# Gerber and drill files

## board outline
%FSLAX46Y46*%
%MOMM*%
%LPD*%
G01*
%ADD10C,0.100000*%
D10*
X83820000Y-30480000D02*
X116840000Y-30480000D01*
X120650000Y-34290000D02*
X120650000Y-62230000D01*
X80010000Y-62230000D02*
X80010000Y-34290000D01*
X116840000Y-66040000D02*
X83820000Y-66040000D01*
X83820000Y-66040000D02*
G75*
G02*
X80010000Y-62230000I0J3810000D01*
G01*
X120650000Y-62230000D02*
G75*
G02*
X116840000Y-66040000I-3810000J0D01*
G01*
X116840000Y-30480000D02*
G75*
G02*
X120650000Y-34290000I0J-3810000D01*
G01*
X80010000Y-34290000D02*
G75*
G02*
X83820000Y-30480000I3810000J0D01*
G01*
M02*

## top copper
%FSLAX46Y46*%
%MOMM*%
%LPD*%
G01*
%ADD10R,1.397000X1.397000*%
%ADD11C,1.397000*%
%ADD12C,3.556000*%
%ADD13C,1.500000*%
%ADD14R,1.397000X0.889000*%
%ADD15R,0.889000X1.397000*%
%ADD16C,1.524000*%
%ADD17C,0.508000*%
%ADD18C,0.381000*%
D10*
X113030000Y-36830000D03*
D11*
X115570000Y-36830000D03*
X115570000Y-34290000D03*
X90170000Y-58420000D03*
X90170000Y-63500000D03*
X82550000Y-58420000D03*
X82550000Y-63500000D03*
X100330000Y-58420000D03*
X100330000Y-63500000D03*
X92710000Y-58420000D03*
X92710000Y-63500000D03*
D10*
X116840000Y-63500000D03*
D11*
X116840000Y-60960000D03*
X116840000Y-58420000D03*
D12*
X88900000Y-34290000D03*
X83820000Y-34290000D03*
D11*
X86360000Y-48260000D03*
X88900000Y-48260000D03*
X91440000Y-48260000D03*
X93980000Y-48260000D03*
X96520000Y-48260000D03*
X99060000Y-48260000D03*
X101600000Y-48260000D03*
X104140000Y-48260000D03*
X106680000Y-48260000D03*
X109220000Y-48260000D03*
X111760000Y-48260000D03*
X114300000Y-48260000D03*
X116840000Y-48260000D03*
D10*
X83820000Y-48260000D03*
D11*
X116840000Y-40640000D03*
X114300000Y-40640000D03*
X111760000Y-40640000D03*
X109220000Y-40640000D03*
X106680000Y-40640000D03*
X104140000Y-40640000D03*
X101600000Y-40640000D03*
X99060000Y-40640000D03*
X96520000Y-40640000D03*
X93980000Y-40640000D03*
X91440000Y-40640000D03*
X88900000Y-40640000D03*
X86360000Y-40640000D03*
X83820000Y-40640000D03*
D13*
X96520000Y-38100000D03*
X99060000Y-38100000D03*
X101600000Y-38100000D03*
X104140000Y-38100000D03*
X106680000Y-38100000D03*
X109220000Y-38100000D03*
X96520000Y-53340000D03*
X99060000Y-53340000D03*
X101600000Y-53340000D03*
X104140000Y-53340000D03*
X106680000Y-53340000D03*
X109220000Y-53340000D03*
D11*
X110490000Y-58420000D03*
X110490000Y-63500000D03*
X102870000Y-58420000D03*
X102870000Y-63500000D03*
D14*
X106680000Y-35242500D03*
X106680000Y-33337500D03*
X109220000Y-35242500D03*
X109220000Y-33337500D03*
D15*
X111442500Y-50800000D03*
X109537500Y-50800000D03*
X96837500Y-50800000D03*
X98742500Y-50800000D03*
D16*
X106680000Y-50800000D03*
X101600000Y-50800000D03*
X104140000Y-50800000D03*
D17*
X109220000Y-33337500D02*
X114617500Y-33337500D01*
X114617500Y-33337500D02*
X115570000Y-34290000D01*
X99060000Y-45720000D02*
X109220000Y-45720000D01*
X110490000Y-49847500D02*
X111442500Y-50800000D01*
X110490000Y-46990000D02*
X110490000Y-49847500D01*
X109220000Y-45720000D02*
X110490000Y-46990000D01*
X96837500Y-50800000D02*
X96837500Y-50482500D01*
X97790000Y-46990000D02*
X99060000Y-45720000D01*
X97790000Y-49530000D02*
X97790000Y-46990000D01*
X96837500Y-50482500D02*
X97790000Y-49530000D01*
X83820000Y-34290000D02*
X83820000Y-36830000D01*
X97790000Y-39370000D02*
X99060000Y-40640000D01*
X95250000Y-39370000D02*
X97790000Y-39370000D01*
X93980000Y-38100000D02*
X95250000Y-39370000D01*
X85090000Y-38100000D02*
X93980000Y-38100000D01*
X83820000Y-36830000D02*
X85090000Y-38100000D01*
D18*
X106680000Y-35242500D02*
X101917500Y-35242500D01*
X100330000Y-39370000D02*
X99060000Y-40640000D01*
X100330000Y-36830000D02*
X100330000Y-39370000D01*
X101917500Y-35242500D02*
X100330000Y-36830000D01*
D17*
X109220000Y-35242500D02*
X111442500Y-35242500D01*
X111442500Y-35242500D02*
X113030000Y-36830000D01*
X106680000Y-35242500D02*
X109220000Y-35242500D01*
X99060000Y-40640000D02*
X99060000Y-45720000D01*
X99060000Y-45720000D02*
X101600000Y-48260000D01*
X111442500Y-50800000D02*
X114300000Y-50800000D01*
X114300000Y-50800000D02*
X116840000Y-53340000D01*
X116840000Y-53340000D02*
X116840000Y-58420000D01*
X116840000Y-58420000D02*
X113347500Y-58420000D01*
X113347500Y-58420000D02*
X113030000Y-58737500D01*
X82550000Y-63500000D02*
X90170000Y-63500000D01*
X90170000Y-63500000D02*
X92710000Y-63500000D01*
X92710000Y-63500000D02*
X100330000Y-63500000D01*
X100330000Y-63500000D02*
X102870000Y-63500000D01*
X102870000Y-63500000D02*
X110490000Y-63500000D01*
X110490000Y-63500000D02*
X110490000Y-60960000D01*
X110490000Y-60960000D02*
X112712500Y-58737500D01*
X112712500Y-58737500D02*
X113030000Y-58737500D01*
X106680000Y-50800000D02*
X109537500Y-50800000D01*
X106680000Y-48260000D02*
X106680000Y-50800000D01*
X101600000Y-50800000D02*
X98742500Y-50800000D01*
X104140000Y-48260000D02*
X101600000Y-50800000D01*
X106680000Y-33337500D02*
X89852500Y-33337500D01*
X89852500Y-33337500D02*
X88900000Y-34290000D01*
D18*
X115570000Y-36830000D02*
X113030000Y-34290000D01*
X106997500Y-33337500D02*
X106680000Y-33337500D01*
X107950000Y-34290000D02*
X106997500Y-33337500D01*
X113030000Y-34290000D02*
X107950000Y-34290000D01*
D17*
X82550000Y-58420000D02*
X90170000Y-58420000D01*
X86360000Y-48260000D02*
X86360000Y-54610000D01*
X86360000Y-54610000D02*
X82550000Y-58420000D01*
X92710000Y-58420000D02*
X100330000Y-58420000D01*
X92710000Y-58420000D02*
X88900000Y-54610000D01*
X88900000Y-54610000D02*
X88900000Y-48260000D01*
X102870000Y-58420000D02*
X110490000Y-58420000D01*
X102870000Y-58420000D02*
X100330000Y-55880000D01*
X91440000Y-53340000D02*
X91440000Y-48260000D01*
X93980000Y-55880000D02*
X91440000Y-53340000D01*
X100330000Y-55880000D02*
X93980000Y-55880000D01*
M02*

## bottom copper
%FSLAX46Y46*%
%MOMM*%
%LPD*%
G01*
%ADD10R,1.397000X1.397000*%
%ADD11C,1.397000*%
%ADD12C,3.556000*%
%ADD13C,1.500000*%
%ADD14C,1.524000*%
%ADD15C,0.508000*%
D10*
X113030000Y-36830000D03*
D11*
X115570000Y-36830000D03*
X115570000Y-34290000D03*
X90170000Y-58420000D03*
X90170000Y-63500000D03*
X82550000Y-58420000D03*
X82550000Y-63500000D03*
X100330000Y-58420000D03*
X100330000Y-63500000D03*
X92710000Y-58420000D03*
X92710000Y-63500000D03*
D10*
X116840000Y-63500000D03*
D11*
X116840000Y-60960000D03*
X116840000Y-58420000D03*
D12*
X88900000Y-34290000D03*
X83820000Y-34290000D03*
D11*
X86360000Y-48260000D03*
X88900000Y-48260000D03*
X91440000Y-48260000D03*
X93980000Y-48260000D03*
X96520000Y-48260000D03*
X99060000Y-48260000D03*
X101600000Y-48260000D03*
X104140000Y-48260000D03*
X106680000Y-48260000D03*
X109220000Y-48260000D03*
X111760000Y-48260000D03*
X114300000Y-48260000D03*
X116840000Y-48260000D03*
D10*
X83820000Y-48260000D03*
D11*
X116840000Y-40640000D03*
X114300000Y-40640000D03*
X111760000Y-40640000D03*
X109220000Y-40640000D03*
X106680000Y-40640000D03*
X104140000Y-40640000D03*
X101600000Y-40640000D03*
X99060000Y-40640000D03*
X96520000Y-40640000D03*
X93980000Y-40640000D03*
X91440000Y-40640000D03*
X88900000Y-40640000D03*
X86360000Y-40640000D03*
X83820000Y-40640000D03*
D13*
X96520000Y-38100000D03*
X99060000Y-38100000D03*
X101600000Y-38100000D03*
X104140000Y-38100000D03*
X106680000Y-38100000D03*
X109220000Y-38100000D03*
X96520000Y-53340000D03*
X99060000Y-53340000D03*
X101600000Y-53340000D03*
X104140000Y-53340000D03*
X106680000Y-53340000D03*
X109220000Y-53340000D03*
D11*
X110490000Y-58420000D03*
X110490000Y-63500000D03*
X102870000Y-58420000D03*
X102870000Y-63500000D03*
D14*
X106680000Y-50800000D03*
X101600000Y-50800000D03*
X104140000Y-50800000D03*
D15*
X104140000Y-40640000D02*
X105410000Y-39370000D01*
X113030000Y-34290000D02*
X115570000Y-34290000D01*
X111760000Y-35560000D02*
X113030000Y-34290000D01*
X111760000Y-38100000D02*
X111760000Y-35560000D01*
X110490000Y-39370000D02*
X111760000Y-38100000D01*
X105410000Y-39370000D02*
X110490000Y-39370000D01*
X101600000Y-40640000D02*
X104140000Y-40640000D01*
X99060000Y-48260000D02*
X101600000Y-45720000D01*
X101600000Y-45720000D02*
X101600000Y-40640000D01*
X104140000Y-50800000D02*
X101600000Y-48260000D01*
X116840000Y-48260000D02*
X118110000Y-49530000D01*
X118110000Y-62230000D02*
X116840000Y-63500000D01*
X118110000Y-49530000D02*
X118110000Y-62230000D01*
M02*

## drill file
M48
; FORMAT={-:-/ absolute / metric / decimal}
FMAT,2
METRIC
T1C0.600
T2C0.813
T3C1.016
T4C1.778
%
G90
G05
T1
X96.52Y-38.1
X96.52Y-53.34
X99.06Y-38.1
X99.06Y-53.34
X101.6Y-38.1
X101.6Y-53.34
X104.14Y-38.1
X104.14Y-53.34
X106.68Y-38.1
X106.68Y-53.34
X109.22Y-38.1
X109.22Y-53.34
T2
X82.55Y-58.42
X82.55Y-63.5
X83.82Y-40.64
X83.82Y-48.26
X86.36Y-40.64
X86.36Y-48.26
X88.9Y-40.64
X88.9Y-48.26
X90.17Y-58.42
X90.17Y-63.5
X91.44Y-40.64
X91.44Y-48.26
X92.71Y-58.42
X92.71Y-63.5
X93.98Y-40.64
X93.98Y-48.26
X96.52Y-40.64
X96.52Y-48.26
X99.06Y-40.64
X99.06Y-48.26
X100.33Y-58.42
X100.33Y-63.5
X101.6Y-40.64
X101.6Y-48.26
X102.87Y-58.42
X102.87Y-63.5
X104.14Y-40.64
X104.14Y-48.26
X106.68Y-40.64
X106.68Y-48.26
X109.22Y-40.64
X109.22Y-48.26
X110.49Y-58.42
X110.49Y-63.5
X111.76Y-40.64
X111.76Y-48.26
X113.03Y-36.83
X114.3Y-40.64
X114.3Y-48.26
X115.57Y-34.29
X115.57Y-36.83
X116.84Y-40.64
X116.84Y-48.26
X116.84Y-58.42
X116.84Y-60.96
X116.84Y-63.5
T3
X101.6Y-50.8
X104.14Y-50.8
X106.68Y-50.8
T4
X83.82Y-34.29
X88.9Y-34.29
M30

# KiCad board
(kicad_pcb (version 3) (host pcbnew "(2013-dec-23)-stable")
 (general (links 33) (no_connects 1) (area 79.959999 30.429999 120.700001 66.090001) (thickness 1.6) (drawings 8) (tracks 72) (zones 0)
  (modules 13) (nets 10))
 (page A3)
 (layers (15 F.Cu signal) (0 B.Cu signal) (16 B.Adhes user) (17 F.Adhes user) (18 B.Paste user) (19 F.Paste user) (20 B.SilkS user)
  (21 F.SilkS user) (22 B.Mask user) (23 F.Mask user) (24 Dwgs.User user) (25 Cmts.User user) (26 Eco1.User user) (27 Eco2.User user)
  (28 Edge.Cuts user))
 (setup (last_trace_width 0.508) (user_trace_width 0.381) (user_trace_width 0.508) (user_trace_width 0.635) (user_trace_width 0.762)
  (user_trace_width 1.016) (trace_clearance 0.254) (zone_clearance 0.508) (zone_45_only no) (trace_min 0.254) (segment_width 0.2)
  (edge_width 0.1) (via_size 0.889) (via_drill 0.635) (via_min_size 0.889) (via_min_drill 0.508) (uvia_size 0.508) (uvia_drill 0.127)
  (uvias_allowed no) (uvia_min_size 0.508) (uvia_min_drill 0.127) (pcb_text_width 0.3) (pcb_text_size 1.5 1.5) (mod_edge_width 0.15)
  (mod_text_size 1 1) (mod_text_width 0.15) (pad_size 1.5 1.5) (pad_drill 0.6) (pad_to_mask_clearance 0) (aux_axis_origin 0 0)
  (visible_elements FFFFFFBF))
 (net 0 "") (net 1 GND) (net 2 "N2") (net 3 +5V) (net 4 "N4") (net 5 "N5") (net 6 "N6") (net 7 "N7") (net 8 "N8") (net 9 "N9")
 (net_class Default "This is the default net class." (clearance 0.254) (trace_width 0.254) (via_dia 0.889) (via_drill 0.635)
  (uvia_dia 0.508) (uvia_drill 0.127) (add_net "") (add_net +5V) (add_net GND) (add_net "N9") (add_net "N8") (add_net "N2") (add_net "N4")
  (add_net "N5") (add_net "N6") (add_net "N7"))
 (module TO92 (layer F.Cu) (at 114.3 35.56 180)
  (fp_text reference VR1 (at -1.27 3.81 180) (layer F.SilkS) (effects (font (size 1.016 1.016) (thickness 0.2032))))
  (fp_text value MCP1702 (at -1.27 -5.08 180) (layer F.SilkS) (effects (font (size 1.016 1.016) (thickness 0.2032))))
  (pad 1 thru_hole rect (at 1.27 -1.27 180) (size 1.397 1.397) (drill 0.8128) (layers *.Cu *.Mask F.SilkS) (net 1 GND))
  (pad 2 thru_hole circle (at -1.27 -1.27 180) (size 1.397 1.397) (drill 0.8128) (layers *.Cu *.Mask F.SilkS) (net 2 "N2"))
  (pad 3 thru_hole circle (at -1.27 1.27 180) (size 1.397 1.397) (drill 0.8128) (layers *.Cu *.Mask F.SilkS) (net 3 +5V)))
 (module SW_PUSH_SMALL (layer F.Cu) (at 86.36 60.96)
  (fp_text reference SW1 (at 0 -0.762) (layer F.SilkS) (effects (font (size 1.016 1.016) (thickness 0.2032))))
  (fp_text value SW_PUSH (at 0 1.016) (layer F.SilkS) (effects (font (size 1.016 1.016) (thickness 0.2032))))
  (pad 1 thru_hole circle (at 3.81 -2.54) (size 1.397 1.397) (drill 0.8128) (layers *.Cu *.Mask F.SilkS) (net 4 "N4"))
  (pad 2 thru_hole circle (at 3.81 2.54) (size 1.397 1.397) (drill 0.8128) (layers *.Cu *.Mask F.SilkS) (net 1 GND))
  (pad 1 thru_hole circle (at -3.81 -2.54) (size 1.397 1.397) (drill 0.8128) (layers *.Cu *.Mask F.SilkS) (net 4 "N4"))
  (pad 2 thru_hole circle (at -3.81 2.54) (size 1.397 1.397) (drill 0.8128) (layers *.Cu *.Mask F.SilkS) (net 1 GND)))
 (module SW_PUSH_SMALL (layer F.Cu) (at 96.52 60.96)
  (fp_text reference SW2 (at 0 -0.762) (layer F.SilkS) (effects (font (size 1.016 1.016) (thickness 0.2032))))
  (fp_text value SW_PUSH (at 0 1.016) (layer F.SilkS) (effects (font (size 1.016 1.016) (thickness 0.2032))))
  (pad 1 thru_hole circle (at 3.81 -2.54) (size 1.397 1.397) (drill 0.8128) (layers *.Cu *.Mask F.SilkS) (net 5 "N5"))
  (pad 2 thru_hole circle (at 3.81 2.54) (size 1.397 1.397) (drill 0.8128) (layers *.Cu *.Mask F.SilkS) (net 1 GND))
  (pad 1 thru_hole circle (at -3.81 -2.54) (size 1.397 1.397) (drill 0.8128) (layers *.Cu *.Mask F.SilkS) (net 5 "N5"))
  (pad 2 thru_hole circle (at -3.81 2.54) (size 1.397 1.397) (drill 0.8128) (layers *.Cu *.Mask F.SilkS) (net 1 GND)))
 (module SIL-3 (layer F.Cu) (at 116.84 60.96 90)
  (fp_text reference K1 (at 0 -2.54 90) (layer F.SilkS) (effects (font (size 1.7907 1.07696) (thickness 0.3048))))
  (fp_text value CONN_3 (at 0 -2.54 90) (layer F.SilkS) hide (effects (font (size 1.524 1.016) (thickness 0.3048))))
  (pad 1 thru_hole rect (at -2.54 0 90) (size 1.397 1.397) (drill 0.8128) (layers *.Cu *.Mask F.SilkS) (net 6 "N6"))
  (pad 2 thru_hole circle (at 0 0 90) (size 1.397 1.397) (drill 0.8128) (layers *.Cu *.Mask F.SilkS) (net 3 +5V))
  (pad 3 thru_hole circle (at 2.54 0 90) (size 1.397 1.397) (drill 0.8128) (layers *.Cu *.Mask F.SilkS) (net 1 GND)))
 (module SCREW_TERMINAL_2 (layer F.Cu) (at 86.36 34.29 180)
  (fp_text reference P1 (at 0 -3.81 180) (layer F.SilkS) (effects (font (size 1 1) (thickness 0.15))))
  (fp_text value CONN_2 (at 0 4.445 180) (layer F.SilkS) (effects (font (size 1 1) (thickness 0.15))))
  (pad 1 thru_hole circle (at -2.54 0 180) (size 3.556 3.556) (drill 1.778) (layers *.Cu *.Mask F.SilkS) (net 2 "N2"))
  (pad 2 thru_hole circle (at 2.54 0 180) (size 3.556 3.556) (drill 1.778) (layers *.Cu *.Mask F.SilkS) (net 1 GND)))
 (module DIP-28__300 (layer F.Cu) (at 100.33 44.45)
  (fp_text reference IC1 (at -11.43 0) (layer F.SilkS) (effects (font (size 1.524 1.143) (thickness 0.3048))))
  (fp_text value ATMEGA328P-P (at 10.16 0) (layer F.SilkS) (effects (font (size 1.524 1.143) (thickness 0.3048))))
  (pad 2 thru_hole circle (at -13.97 3.81) (size 1.397 1.397) (drill 0.8128) (layers *.Cu *.Mask F.SilkS) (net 4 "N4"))
  (pad 3 thru_hole circle (at -11.43 3.81) (size 1.397 1.397) (drill 0.8128) (layers *.Cu *.Mask F.SilkS) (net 5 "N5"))
  (pad 4 thru_hole circle (at -8.89 3.81) (size 1.397 1.397) (drill 0.8128) (layers *.Cu *.Mask F.SilkS) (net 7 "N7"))
  (pad 5 thru_hole circle (at -6.35 3.81) (size 1.397 1.397) (drill 0.8128) (layers *.Cu *.Mask F.SilkS))
  (pad 6 thru_hole circle (at -3.81 3.81) (size 1.397 1.397) (drill 0.8128) (layers *.Cu *.Mask F.SilkS))
  (pad 7 thru_hole circle (at -1.27 3.81) (size 1.397 1.397) (drill 0.8128) (layers *.Cu *.Mask F.SilkS) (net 3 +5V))
  (pad 8 thru_hole circle (at 1.27 3.81) (size 1.397 1.397) (drill 0.8128) (layers *.Cu *.Mask F.SilkS) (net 1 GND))
  (pad 9 thru_hole circle (at 3.81 3.81) (size 1.397 1.397) (drill 0.8128) (layers *.Cu *.Mask F.SilkS) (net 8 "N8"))
  (pad 10 thru_hole circle (at 6.35 3.81) (size 1.397 1.397) (drill 0.8128) (layers *.Cu *.Mask F.SilkS) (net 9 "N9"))
  (pad 11 thru_hole circle (at 8.89 3.81) (size 1.397 1.397) (drill 0.8128) (layers *.Cu *.Mask F.SilkS))
  (pad 12 thru_hole circle (at 11.43 3.81) (size 1.397 1.397) (drill 0.8128) (layers *.Cu *.Mask F.SilkS))
  (pad 13 thru_hole circle (at 13.97 3.81) (size 1.397 1.397) (drill 0.8128) (layers *.Cu *.Mask F.SilkS))
  (pad 14 thru_hole circle (at 16.51 3.81) (size 1.397 1.397) (drill 0.8128) (layers *.Cu *.Mask F.SilkS) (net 6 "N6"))
  (pad 1 thru_hole rect (at -16.51 3.81) (size 1.397 1.397) (drill 0.8128) (layers *.Cu *.Mask F.SilkS))
  (pad 15 thru_hole circle (at 16.51 -3.81) (size 1.397 1.397) (drill 0.8128) (layers *.Cu *.Mask F.SilkS))
  (pad 16 thru_hole circle (at 13.97 -3.81) (size 1.397 1.397) (drill 0.8128) (layers *.Cu *.Mask F.SilkS))
  (pad 17 thru_hole circle (at 11.43 -3.81) (size 1.397 1.397) (drill 0.8128) (layers *.Cu *.Mask F.SilkS))
  (pad 18 thru_hole circle (at 8.89 -3.81) (size 1.397 1.397) (drill 0.8128) (layers *.Cu *.Mask F.SilkS))
  (pad 19 thru_hole circle (at 6.35 -3.81) (size 1.397 1.397) (drill 0.8128) (layers *.Cu *.Mask F.SilkS))
  (pad 20 thru_hole circle (at 3.81 -3.81) (size 1.397 1.397) (drill 0.8128) (layers *.Cu *.Mask F.SilkS) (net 3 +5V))
  (pad 21 thru_hole circle (at 1.27 -3.81) (size 1.397 1.397) (drill 0.8128) (layers *.Cu *.Mask F.SilkS) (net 3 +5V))
  (pad 22 thru_hole circle (at -1.27 -3.81) (size 1.397 1.397) (drill 0.8128) (layers *.Cu *.Mask F.SilkS) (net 1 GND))
  (pad 23 thru_hole circle (at -3.81 -3.81) (size 1.397 1.397) (drill 0.8128) (layers *.Cu *.Mask F.SilkS))
  (pad 24 thru_hole circle (at -6.35 -3.81) (size 1.397 1.397) (drill 0.8128) (layers *.Cu *.Mask F.SilkS))
  (pad 25 thru_hole circle (at -8.89 -3.81) (size 1.397 1.397) (drill 0.8128) (layers *.Cu *.Mask F.SilkS))
  (pad 26 thru_hole circle (at -11.43 -3.81) (size 1.397 1.397) (drill 0.8128) (layers *.Cu *.Mask F.SilkS))
  (pad 27 thru_hole circle (at -13.97 -3.81) (size 1.397 1.397) (drill 0.8128) (layers *.Cu *.Mask F.SilkS))
  (pad 28 thru_hole circle (at -16.51 -3.81) (size 1.397 1.397) (drill 0.8128) (layers *.Cu *.Mask F.SilkS)))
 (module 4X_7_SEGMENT (layer F.Cu) (at 104.14 45.72)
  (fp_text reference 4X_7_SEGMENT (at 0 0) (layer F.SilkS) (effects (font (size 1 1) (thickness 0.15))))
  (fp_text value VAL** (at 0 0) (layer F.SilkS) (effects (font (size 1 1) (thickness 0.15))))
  (pad 1 thru_hole circle (at -7.62 -7.62) (size 1.5 1.5) (drill 0.6) (layers *.Cu *.Mask F.SilkS))
  (pad 2 thru_hole circle (at -5.08 -7.62) (size 1.5 1.5) (drill 0.6) (layers *.Cu *.Mask F.SilkS))
  (pad 3 thru_hole circle (at -2.54 -7.62) (size 1.5 1.5) (drill 0.6) (layers *.Cu *.Mask F.SilkS))
  (pad 4 thru_hole circle (at 0 -7.62) (size 1.5 1.5) (drill 0.6) (layers *.Cu *.Mask F.SilkS))
  (pad 5 thru_hole circle (at 2.54 -7.62) (size 1.5 1.5) (drill 0.6) (layers *.Cu *.Mask F.SilkS))
  (pad 6 thru_hole circle (at 5.08 -7.62) (size 1.5 1.5) (drill 0.6) (layers *.Cu *.Mask F.SilkS))
  (pad 7 thru_hole circle (at -7.62 7.62) (size 1.5 1.5) (drill 0.6) (layers *.Cu *.Mask F.SilkS))
  (pad 8 thru_hole circle (at -5.08 7.62) (size 1.5 1.5) (drill 0.6) (layers *.Cu *.Mask F.SilkS))
  (pad 9 thru_hole circle (at -2.54 7.62) (size 1.5 1.5) (drill 0.6) (layers *.Cu *.Mask F.SilkS))
  (pad 10 thru_hole circle (at 0 7.62) (size 1.5 1.5) (drill 0.6) (layers *.Cu *.Mask F.SilkS))
  (pad 11 thru_hole circle (at 2.54 7.62) (size 1.5 1.5) (drill 0.6) (layers *.Cu *.Mask F.SilkS))
  (pad 12 thru_hole circle (at 5.08 7.62) (size 1.5 1.5) (drill 0.6) (layers *.Cu *.Mask F.SilkS)))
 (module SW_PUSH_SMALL (layer F.Cu) (at 106.68 60.96)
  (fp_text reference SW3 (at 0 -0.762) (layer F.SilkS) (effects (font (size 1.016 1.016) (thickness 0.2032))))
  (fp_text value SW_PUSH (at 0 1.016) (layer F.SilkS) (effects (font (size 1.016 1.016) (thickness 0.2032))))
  (pad 1 thru_hole circle (at 3.81 -2.54) (size 1.397 1.397) (drill 0.8128) (layers *.Cu *.Mask F.SilkS) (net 7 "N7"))
  (pad 2 thru_hole circle (at 3.81 2.54) (size 1.397 1.397) (drill 0.8128) (layers *.Cu *.Mask F.SilkS) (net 1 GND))
  (pad 1 thru_hole circle (at -3.81 -2.54) (size 1.397 1.397) (drill 0.8128) (layers *.Cu *.Mask F.SilkS) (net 7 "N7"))
  (pad 2 thru_hole circle (at -3.81 2.54) (size 1.397 1.397) (drill 0.8128) (layers *.Cu *.Mask F.SilkS) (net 1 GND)))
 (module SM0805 (layer F.Cu) (at 106.68 34.29 90)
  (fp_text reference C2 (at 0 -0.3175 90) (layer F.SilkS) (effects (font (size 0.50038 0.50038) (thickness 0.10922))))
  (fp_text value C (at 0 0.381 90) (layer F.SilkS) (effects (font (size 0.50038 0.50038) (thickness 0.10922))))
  (pad 1 smd rect (at -0.9525 0 90) (size 0.889 1.397) (layers F.Cu F.Paste F.Mask) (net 1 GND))
  (pad 2 smd rect (at 0.9525 0 90) (size 0.889 1.397) (layers F.Cu F.Paste F.Mask) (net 2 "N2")))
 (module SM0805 (layer F.Cu) (at 109.22 34.29 90)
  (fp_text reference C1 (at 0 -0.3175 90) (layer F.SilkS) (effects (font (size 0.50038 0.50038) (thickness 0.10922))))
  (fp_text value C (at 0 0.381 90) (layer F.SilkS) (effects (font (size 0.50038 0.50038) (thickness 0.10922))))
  (pad 1 smd rect (at -0.9525 0 90) (size 0.889 1.397) (layers F.Cu F.Paste F.Mask) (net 1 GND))
  (pad 2 smd rect (at 0.9525 0 90) (size 0.889 1.397) (layers F.Cu F.Paste F.Mask) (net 3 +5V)))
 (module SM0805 (layer F.Cu) (at 110.49 50.8 180)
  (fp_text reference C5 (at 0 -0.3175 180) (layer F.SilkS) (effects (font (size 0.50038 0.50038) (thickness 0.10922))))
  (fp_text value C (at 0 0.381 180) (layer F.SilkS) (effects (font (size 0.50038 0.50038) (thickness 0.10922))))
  (pad 1 smd rect (at -0.9525 0 180) (size 0.889 1.397) (layers F.Cu F.Paste F.Mask) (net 1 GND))
  (pad 2 smd rect (at 0.9525 0 180) (size 0.889 1.397) (layers F.Cu F.Paste F.Mask) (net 9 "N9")))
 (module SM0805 (layer F.Cu) (at 97.79 50.8)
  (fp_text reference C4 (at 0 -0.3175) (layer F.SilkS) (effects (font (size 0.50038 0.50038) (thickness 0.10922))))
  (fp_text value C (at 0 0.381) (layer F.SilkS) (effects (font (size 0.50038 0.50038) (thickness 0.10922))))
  (pad 1 smd rect (at -0.9525 0) (size 0.889 1.397) (layers F.Cu F.Paste F.Mask) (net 1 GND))
  (pad 2 smd rect (at 0.9525 0) (size 0.889 1.397) (layers F.Cu F.Paste F.Mask) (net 8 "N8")))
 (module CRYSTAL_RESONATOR (layer F.Cu) (at 104.14 50.8 180)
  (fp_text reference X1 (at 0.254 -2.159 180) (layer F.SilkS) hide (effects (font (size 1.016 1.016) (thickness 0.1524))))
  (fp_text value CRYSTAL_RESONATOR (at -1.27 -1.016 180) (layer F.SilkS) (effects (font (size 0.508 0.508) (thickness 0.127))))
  (pad 1 thru_hole circle (at -2.54 0 180) (size 1.524 1.524) (drill 1.016) (layers *.Cu *.Mask F.SilkS) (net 9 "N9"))
  (pad 2 thru_hole circle (at 2.54 0 180) (size 1.524 1.524) (drill 1.016) (layers *.Cu *.Mask F.SilkS) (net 8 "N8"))
  (pad 3 thru_hole circle (at 0 0 180) (size 1.524 1.524) (drill 1.016) (layers *.Cu *.Mask F.SilkS) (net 1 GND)))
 (gr_line (start 83.82 30.48) (end 116.84 30.48) (angle 90) (layer Edge.Cuts) (width 0.1))
 (gr_line (start 120.65 34.29) (end 120.65 62.23) (angle 90) (layer Edge.Cuts) (width 0.1))
 (gr_line (start 80.01 62.23) (end 80.01 34.29) (angle 90) (layer Edge.Cuts) (width 0.1))
 (gr_line (start 116.84 66.04) (end 83.82 66.04) (angle 90) (layer Edge.Cuts) (width 0.1))
 (gr_arc (start 83.82 62.23) (end 83.82 66.04) (angle 90) (layer Edge.Cuts) (width 0.1))
 (gr_arc (start 116.84 62.23) (end 120.65 62.23) (angle 90) (layer Edge.Cuts) (width 0.1))
 (gr_arc (start 116.84 34.29) (end 116.84 30.48) (angle 90) (layer Edge.Cuts) (width 0.1))
 (gr_arc (start 83.82 34.29) (end 80.01 34.29) (angle 90) (layer Edge.Cuts) (width 0.1))
 (segment (start 104.14 40.64) (end 105.41 39.37) (width 0.508) (layer B.Cu) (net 3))
 (segment (start 113.03 34.29) (end 115.57 34.29) (width 0.508) (layer B.Cu) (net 3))
 (segment (start 111.76 35.56) (end 113.03 34.29) (width 0.508) (layer B.Cu) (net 3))
 (segment (start 111.76 38.1) (end 111.76 35.56) (width 0.508) (layer B.Cu) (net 3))
 (segment (start 110.49 39.37) (end 111.76 38.1) (width 0.508) (layer B.Cu) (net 3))
 (segment (start 105.41 39.37) (end 110.49 39.37) (width 0.508) (layer B.Cu) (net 3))
 (segment (start 109.22 33.3375) (end 114.6175 33.3375) (width 0.508) (layer F.Cu) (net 3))
 (segment (start 114.6175 33.3375) (end 115.57 34.29) (width 0.508) (layer F.Cu) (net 3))
 (segment (start 101.6 40.64) (end 104.14 40.64) (width 0.508) (layer B.Cu) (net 3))
 (segment (start 99.06 48.26) (end 101.6 45.72) (width 0.508) (layer B.Cu) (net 3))
 (segment (start 101.6 45.72) (end 101.6 40.64) (width 0.508) (layer B.Cu) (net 3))
 (segment (start 99.06 45.72) (end 109.22 45.72) (width 0.508) (layer F.Cu) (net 1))
 (segment (start 110.49 49.8475) (end 111.4425 50.8) (width 0.508) (layer F.Cu) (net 1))
 (segment (start 110.49 46.99) (end 110.49 49.8475) (width 0.508) (layer F.Cu) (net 1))
 (segment (start 109.22 45.72) (end 110.49 46.99) (width 0.508) (layer F.Cu) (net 1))
 (segment (start 96.8375 50.8) (end 96.8375 50.4825) (width 0.508) (layer F.Cu) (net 1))
 (segment (start 97.79 46.99) (end 99.06 45.72) (width 0.508) (layer F.Cu) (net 1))
 (segment (start 97.79 49.53) (end 97.79 46.99) (width 0.508) (layer F.Cu) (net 1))
 (segment (start 96.8375 50.4825) (end 97.79 49.53) (width 0.508) (layer F.Cu) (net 1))
 (segment (start 83.82 34.29) (end 83.82 36.83) (width 0.508) (layer F.Cu) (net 1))
 (segment (start 97.79 39.37) (end 99.06 40.64) (width 0.508) (layer F.Cu) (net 1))
 (segment (start 95.25 39.37) (end 97.79 39.37) (width 0.508) (layer F.Cu) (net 1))
 (segment (start 93.98 38.1) (end 95.25 39.37) (width 0.508) (layer F.Cu) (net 1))
 (segment (start 85.09 38.1) (end 93.98 38.1) (width 0.508) (layer F.Cu) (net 1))
 (segment (start 83.82 36.83) (end 85.09 38.1) (width 0.508) (layer F.Cu) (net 1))
 (segment (start 106.68 35.2425) (end 101.9175 35.2425) (width 0.381) (layer F.Cu) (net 1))
 (segment (start 100.33 39.37) (end 99.06 40.64) (width 0.381) (layer F.Cu) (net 1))
 (segment (start 100.33 36.83) (end 100.33 39.37) (width 0.381) (layer F.Cu) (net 1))
 (segment (start 101.9175 35.2425) (end 100.33 36.83) (width 0.381) (layer F.Cu) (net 1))
 (segment (start 109.22 35.2425) (end 111.4425 35.2425) (width 0.508) (layer F.Cu) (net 1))
 (segment (start 111.4425 35.2425) (end 113.03 36.83) (width 0.508) (layer F.Cu) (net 1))
 (segment (start 106.68 35.2425) (end 109.22 35.2425) (width 0.508) (layer F.Cu) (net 1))
 (segment (start 99.06 40.64) (end 99.06 45.72) (width 0.508) (layer F.Cu) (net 1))
 (segment (start 99.06 45.72) (end 101.6 48.26) (width 0.508) (layer F.Cu) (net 1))
 (segment (start 104.14 50.8) (end 101.6 48.26) (width 0.508) (layer B.Cu) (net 1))
 (segment (start 111.4425 50.8) (end 114.3 50.8) (width 0.508) (layer F.Cu) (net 1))
 (segment (start 114.3 50.8) (end 116.84 53.34) (width 0.508) (layer F.Cu) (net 1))
 (segment (start 116.84 53.34) (end 116.84 58.42) (width 0.508) (layer F.Cu) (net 1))
 (segment (start 116.84 58.42) (end 113.3475 58.42) (width 0.508) (layer F.Cu) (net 1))
 (segment (start 113.3475 58.42) (end 113.03 58.7375) (width 0.508) (layer F.Cu) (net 1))
 (segment (start 82.55 63.5) (end 90.17 63.5) (width 0.508) (layer F.Cu) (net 1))
 (segment (start 90.17 63.5) (end 92.71 63.5) (width 0.508) (layer F.Cu) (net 1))
 (segment (start 92.71 63.5) (end 100.33 63.5) (width 0.508) (layer F.Cu) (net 1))
 (segment (start 100.33 63.5) (end 102.87 63.5) (width 0.508) (layer F.Cu) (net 1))
 (segment (start 102.87 63.5) (end 110.49 63.5) (width 0.508) (layer F.Cu) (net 1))
 (segment (start 110.49 63.5) (end 110.49 60.96) (width 0.508) (layer F.Cu) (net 1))
 (segment (start 110.49 60.96) (end 112.7125 58.7375) (width 0.508) (layer F.Cu) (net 1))
 (segment (start 112.7125 58.7375) (end 113.03 58.7375) (width 0.508) (layer F.Cu) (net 1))
 (segment (start 106.68 50.8) (end 109.5375 50.8) (width 0.508) (layer F.Cu) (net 9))
 (segment (start 106.68 48.26) (end 106.68 50.8) (width 0.508) (layer F.Cu) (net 9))
 (segment (start 101.6 50.8) (end 98.7425 50.8) (width 0.508) (layer F.Cu) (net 8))
 (segment (start 104.14 48.26) (end 101.6 50.8) (width 0.508) (layer F.Cu) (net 8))
 (segment (start 106.68 33.3375) (end 89.8525 33.3375) (width 0.508) (layer F.Cu) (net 2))
 (segment (start 89.8525 33.3375) (end 88.9 34.29) (width 0.508) (layer F.Cu) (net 2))
 (segment (start 115.57 36.83) (end 113.03 34.29) (width 0.381) (layer F.Cu) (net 2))
 (segment (start 106.9975 33.3375) (end 106.68 33.3375) (width 0.381) (layer F.Cu) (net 2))
 (segment (start 107.95 34.29) (end 106.9975 33.3375) (width 0.381) (layer F.Cu) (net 2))
 (segment (start 113.03 34.29) (end 107.95 34.29) (width 0.381) (layer F.Cu) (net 2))
 (segment (start 82.55 58.42) (end 90.17 58.42) (width 0.508) (layer F.Cu) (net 4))
 (segment (start 86.36 48.26) (end 86.36 54.61) (width 0.508) (layer F.Cu) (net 4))
 (segment (start 86.36 54.61) (end 82.55 58.42) (width 0.508) (layer F.Cu) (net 4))
 (segment (start 92.71 58.42) (end 100.33 58.42) (width 0.508) (layer F.Cu) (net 5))
 (segment (start 92.71 58.42) (end 88.9 54.61) (width 0.508) (layer F.Cu) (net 5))
 (segment (start 88.9 54.61) (end 88.9 48.26) (width 0.508) (layer F.Cu) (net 5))
 (segment (start 116.84 48.26) (end 118.11 49.53) (width 0.508) (layer B.Cu) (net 6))
 (segment (start 118.11 62.23) (end 116.84 63.5) (width 0.508) (layer B.Cu) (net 6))
 (segment (start 118.11 49.53) (end 118.11 62.23) (width 0.508) (layer B.Cu) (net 6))
 (segment (start 102.87 58.42) (end 110.49 58.42) (width 0.508) (layer F.Cu) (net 7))
 (segment (start 102.87 58.42) (end 100.33 55.88) (width 0.508) (layer F.Cu) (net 7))
 (segment (start 91.44 53.34) (end 91.44 48.26) (width 0.508) (layer F.Cu) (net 7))
 (segment (start 93.98 55.88) (end 91.44 53.34) (width 0.508) (layer F.Cu) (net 7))
 (segment (start 100.33 55.88) (end 93.98 55.88) (width 0.508) (layer F.Cu) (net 7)))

